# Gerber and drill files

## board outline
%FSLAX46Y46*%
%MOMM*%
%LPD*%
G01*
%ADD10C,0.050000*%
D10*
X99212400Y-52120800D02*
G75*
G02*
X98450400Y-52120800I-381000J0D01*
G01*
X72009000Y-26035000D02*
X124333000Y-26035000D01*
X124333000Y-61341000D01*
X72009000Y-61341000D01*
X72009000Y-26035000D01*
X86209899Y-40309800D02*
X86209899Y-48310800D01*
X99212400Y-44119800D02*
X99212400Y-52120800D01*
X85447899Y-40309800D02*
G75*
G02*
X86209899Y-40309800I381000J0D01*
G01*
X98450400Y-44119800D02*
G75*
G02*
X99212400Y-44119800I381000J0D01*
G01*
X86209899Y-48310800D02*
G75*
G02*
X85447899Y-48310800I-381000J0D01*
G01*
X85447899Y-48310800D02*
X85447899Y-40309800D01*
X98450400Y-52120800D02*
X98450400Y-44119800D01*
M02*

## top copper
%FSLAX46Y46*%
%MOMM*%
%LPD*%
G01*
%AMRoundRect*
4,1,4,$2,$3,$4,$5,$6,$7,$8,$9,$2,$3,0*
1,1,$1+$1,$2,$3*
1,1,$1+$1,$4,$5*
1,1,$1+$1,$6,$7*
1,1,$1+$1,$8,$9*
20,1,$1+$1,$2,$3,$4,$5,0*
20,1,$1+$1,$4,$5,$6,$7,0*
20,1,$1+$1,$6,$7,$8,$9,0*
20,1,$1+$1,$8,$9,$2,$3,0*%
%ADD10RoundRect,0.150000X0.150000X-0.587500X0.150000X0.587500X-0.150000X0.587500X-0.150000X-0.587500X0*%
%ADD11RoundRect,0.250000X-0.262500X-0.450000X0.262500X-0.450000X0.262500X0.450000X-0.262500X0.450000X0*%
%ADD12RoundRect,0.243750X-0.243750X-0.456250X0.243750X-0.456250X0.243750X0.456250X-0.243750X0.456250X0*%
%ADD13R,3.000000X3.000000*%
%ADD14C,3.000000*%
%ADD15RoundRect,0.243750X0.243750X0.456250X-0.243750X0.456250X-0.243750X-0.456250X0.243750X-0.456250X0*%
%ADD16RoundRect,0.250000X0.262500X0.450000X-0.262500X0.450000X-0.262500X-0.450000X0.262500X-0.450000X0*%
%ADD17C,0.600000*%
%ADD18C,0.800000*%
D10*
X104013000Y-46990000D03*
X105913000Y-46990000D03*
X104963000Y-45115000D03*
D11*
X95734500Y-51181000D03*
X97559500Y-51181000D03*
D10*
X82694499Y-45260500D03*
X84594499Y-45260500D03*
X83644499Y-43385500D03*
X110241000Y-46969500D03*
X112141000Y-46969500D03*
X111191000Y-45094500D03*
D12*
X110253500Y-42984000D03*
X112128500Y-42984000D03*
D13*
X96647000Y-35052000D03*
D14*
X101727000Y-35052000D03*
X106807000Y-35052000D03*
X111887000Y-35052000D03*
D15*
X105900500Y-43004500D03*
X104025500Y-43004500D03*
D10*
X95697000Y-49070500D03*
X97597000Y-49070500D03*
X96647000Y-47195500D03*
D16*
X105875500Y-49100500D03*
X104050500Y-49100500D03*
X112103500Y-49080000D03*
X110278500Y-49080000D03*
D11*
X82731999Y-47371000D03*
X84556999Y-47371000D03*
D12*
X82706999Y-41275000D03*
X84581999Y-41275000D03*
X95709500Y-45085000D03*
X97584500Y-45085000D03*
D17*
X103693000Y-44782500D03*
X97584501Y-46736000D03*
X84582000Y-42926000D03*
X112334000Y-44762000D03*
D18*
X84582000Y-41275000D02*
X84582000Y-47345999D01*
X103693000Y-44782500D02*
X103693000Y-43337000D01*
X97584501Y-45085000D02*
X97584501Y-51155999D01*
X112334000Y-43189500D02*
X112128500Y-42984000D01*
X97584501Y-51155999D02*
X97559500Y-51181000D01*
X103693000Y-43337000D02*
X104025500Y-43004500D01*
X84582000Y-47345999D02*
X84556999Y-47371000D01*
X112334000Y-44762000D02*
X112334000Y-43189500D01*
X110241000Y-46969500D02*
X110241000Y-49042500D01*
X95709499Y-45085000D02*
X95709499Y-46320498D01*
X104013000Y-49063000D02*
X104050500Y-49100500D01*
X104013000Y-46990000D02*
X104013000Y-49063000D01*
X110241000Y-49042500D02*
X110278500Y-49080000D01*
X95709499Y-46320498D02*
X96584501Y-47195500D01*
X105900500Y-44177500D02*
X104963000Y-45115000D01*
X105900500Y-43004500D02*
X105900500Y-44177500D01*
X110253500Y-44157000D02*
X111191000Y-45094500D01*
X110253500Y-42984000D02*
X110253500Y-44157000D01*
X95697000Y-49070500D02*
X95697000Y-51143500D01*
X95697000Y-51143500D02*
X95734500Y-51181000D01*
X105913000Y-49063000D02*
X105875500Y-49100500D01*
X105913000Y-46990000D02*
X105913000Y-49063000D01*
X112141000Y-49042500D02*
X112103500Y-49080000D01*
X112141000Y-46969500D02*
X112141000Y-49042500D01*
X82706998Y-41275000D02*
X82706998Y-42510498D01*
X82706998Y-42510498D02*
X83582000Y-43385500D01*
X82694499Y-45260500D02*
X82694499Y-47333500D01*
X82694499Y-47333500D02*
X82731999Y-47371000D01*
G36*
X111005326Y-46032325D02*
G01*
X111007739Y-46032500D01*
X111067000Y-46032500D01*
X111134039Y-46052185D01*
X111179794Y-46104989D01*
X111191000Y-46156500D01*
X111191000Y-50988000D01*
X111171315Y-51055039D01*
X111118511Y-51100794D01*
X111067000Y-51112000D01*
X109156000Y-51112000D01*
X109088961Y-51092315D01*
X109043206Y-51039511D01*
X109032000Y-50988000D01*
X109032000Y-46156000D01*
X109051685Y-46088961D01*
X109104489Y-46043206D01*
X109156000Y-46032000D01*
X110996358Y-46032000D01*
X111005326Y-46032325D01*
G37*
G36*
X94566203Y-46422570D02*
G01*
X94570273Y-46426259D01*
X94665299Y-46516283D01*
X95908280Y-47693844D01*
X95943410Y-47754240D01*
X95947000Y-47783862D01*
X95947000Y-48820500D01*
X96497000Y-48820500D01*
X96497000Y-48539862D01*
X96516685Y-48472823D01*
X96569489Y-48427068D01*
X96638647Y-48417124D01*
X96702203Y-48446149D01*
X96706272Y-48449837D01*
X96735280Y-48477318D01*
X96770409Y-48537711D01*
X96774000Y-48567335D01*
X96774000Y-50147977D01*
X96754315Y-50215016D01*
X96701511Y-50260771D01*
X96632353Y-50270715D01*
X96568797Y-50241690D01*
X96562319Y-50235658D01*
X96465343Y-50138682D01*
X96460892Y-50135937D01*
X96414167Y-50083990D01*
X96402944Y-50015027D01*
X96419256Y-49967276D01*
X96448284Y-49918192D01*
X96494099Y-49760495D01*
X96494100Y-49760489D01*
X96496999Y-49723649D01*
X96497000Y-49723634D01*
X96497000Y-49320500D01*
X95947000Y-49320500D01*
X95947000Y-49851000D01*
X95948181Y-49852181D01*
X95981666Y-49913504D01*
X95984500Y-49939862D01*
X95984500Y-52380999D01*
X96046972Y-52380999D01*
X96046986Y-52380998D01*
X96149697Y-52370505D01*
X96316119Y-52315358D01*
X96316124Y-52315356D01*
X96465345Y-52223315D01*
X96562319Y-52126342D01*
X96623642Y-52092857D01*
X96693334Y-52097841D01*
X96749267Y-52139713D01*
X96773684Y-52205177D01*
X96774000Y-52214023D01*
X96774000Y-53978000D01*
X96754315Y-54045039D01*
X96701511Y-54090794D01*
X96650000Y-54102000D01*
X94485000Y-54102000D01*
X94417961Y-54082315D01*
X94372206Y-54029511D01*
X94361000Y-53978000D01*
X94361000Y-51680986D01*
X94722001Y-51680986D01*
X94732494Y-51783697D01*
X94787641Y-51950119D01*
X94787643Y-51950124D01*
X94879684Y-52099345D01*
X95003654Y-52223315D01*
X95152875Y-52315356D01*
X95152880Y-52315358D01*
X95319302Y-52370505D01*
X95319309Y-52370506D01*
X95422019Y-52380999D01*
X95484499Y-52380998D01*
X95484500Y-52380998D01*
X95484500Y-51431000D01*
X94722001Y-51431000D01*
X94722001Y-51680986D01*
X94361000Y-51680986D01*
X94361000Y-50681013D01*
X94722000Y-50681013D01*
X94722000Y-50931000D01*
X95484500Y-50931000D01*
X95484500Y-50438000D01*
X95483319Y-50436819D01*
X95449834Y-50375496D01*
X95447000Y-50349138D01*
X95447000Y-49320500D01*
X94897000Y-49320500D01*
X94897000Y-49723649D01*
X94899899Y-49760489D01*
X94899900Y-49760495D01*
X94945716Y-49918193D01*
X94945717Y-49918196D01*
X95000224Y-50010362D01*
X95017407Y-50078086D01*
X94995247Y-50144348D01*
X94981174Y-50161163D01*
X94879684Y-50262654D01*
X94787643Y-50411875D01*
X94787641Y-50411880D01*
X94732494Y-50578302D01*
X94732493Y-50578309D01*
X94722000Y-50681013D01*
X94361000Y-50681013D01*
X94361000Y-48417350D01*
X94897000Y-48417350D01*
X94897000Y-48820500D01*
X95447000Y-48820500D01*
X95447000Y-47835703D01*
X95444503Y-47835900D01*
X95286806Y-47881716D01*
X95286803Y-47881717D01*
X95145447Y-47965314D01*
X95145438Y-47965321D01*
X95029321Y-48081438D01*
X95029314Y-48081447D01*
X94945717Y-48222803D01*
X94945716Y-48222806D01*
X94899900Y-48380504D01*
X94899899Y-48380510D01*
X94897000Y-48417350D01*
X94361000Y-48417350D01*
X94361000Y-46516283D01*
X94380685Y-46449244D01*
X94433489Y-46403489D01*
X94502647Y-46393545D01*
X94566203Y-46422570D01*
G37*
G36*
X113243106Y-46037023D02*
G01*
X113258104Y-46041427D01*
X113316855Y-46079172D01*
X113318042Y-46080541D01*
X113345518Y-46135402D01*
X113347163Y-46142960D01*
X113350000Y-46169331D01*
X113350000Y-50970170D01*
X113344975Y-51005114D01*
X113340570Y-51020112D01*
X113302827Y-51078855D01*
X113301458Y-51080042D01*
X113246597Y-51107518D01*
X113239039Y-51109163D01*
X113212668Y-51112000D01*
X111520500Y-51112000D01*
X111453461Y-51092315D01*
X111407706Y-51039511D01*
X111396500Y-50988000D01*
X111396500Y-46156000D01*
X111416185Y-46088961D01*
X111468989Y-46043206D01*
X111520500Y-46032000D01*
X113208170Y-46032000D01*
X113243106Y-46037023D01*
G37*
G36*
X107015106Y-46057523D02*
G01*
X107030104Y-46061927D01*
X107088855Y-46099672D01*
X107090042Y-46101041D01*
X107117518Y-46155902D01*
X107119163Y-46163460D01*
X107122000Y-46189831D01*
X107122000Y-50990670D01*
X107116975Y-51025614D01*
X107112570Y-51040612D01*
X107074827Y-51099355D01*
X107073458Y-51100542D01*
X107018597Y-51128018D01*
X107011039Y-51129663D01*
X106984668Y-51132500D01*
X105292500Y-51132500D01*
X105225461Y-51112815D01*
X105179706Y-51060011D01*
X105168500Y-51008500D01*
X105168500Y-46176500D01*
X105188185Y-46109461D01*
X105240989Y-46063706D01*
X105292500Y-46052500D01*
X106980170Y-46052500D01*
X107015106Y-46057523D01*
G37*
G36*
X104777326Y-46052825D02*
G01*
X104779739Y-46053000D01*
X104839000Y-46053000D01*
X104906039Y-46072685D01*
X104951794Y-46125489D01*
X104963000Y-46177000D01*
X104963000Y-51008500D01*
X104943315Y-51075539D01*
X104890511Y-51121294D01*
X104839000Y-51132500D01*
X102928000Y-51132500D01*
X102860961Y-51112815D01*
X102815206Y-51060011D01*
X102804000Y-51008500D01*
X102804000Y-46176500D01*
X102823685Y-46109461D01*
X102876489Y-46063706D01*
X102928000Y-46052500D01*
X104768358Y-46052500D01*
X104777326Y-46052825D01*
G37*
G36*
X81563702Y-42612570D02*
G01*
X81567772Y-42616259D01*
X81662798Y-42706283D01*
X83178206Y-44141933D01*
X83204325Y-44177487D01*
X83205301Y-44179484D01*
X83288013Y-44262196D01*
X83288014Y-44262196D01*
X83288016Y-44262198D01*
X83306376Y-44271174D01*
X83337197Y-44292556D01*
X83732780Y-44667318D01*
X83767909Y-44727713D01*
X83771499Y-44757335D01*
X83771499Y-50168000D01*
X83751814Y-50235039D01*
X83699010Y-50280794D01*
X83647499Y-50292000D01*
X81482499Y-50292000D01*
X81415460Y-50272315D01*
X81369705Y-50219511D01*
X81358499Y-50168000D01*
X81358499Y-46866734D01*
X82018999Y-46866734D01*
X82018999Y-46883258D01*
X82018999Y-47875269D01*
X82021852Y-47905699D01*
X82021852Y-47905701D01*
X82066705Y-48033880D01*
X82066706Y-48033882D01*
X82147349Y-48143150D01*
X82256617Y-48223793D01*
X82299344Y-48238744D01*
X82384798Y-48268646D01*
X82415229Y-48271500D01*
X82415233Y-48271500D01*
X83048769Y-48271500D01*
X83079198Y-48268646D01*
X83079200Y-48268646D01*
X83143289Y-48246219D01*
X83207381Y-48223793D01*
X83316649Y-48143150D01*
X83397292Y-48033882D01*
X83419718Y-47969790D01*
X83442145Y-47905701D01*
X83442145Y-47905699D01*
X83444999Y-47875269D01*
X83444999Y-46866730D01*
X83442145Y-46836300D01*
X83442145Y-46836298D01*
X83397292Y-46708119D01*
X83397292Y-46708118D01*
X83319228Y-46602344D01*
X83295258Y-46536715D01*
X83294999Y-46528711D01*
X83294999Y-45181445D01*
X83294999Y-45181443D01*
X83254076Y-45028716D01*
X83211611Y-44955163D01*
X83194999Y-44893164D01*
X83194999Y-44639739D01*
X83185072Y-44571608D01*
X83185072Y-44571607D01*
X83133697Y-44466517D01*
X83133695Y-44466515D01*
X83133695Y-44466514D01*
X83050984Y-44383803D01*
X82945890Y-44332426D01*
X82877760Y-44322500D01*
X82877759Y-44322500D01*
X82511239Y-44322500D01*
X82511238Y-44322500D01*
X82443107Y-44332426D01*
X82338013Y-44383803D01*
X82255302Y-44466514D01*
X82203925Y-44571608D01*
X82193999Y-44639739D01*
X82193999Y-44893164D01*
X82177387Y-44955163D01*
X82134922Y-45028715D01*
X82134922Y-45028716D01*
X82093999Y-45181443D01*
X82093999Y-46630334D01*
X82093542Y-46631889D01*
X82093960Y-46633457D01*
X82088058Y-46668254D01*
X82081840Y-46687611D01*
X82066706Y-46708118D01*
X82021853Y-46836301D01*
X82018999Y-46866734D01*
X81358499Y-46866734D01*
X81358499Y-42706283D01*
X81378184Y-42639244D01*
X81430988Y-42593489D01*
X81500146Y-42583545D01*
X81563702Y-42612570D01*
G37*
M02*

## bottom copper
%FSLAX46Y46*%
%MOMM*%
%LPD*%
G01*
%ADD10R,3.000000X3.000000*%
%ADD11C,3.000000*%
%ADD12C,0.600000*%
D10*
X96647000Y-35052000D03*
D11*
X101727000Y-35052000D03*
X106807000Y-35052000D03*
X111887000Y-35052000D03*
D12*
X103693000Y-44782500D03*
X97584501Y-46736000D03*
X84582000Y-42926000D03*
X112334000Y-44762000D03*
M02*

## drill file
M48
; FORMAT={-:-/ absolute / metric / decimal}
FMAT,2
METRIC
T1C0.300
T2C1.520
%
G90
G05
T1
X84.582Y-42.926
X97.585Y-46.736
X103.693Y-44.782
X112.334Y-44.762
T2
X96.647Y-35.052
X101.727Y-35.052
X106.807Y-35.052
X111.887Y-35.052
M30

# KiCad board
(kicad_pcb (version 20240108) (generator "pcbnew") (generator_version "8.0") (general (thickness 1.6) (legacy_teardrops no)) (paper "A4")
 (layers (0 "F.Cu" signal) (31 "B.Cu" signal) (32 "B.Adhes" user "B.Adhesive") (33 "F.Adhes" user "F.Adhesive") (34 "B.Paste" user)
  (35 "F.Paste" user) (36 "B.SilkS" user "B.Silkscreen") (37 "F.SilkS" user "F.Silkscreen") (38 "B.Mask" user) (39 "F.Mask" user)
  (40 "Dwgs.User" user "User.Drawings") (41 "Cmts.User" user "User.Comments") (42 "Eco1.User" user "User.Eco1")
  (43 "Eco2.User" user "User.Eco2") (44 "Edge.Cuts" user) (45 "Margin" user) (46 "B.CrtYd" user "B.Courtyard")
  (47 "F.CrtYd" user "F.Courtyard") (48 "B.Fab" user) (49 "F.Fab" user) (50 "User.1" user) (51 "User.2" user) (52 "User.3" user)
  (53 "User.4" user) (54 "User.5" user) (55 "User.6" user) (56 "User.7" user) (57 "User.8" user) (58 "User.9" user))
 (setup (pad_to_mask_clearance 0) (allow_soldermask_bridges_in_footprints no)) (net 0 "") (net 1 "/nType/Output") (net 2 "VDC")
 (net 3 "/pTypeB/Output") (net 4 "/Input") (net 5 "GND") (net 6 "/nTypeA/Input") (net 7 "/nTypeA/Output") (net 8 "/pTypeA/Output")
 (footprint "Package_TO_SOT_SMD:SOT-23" (layer "F.Cu") (at 104.963 46.0525 90)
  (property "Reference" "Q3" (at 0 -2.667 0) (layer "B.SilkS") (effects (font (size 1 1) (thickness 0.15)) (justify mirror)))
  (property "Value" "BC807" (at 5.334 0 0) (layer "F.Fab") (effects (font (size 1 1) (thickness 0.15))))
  (pad "1" smd roundrect (at -0.9375 -0.95 90) (size 1.475 0.6) (layers "F.Cu" "F.Paste" "F.Mask") (roundrect_rratio 0.25)
   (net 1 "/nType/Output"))
  (pad "2" smd roundrect (at -0.9375 0.95 90) (size 1.475 0.6) (layers "F.Cu" "F.Paste" "F.Mask") (roundrect_rratio 0.25) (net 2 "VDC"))
  (pad "3" smd roundrect (at 0.9375 0 90) (size 1.475 0.6) (layers "F.Cu" "F.Paste" "F.Mask") (roundrect_rratio 0.25)
   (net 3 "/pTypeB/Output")))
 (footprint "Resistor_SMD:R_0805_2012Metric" (layer "F.Cu") (at 96.647 51.181)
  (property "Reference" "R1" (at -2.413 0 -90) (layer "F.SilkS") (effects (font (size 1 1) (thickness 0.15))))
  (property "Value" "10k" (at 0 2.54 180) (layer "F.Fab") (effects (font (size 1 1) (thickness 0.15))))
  (pad "1" smd roundrect (at -0.9125 0) (size 1.025 1.4) (layers "F.Cu" "F.Paste" "F.Mask") (roundrect_rratio 0.243902) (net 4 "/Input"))
  (pad "2" smd roundrect (at 0.9125 0) (size 1.025 1.4) (layers "F.Cu" "F.Paste" "F.Mask") (roundrect_rratio 0.243902) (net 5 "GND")))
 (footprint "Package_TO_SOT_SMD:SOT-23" (layer "F.Cu") (at 83.644499 44.323 90)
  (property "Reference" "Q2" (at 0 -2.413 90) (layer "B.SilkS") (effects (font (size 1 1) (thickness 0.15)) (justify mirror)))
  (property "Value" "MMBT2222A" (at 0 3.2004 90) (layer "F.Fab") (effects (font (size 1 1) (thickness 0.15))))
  (pad "1" smd roundrect (at -0.9375 -0.95 90) (size 1.475 0.6) (layers "F.Cu" "F.Paste" "F.Mask") (roundrect_rratio 0.25)
   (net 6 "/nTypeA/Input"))
  (pad "2" smd roundrect (at -0.9375 0.95 90) (size 1.475 0.6) (layers "F.Cu" "F.Paste" "F.Mask") (roundrect_rratio 0.25) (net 5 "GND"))
  (pad "3" smd roundrect (at 0.9375 0 90) (size 1.475 0.6) (layers "F.Cu" "F.Paste" "F.Mask") (roundrect_rratio 0.25)
   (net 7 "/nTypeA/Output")))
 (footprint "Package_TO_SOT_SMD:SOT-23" (layer "F.Cu") (at 111.191 46.032 90)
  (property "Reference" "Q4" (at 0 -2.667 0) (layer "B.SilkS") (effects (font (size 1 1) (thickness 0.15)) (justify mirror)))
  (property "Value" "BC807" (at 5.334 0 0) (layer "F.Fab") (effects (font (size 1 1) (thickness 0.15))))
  (pad "1" smd roundrect (at -0.9375 -0.95 90) (size 1.475 0.6) (layers "F.Cu" "F.Paste" "F.Mask") (roundrect_rratio 0.25)
   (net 1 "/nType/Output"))
  (pad "2" smd roundrect (at -0.9375 0.95 90) (size 1.475 0.6) (layers "F.Cu" "F.Paste" "F.Mask") (roundrect_rratio 0.25) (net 2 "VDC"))
  (pad "3" smd roundrect (at 0.9375 0 90) (size 1.475 0.6) (layers "F.Cu" "F.Paste" "F.Mask") (roundrect_rratio 0.25)
   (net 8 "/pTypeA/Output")))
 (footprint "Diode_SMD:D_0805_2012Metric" (layer "F.Cu") (at 111.191 42.984)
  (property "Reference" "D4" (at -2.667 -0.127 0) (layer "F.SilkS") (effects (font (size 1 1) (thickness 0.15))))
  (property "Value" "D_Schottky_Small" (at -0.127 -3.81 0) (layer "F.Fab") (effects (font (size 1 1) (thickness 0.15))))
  (pad "1" smd roundrect (at -0.9375 0) (size 0.975 1.4) (layers "F.Cu" "F.Paste" "F.Mask") (roundrect_rratio 0.25) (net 8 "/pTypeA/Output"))
  (pad "2" smd roundrect (at 0.9375 0) (size 0.975 1.4) (layers "F.Cu" "F.Paste" "F.Mask") (roundrect_rratio 0.25) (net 5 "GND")))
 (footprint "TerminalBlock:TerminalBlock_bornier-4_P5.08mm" (layer "F.Cu") (at 96.647 35.052)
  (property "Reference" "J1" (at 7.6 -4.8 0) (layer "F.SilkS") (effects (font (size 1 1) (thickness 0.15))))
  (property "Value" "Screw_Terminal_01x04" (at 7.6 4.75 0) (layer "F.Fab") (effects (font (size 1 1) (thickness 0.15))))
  (pad "1" thru_hole rect (at 0 0) (size 3 3) (drill 1.52) (layers "*.Cu" "*.Mask") (remove_unused_layers no) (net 3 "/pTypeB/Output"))
  (pad "2" thru_hole circle (at 5.08 0) (size 3 3) (drill 1.52) (layers "*.Cu" "*.Mask") (remove_unused_layers no) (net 1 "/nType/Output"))
  (pad "3" thru_hole circle (at 10.16 0) (size 3 3) (drill 1.52) (layers "*.Cu" "*.Mask") (remove_unused_layers no) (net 8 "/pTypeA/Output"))
  (pad "4" thru_hole circle (at 15.24 0) (size 3 3) (drill 1.52) (layers "*.Cu" "*.Mask") (remove_unused_layers no) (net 5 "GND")))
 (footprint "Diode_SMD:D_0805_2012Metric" (layer "F.Cu") (at 104.963 43.0045 180)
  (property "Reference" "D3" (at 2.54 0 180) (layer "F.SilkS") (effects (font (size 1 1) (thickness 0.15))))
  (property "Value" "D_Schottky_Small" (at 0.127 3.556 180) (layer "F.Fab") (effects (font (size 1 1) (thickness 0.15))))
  (pad "1" smd roundrect (at -0.9375 0 180) (size 0.975 1.4) (layers "F.Cu" "F.Paste" "F.Mask") (roundrect_rratio 0.25)
   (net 3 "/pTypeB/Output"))
  (pad "2" smd roundrect (at 0.9375 0 180) (size 0.975 1.4) (layers "F.Cu" "F.Paste" "F.Mask") (roundrect_rratio 0.25) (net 5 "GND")))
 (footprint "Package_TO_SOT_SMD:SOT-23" (layer "F.Cu") (at 96.647 48.133 90)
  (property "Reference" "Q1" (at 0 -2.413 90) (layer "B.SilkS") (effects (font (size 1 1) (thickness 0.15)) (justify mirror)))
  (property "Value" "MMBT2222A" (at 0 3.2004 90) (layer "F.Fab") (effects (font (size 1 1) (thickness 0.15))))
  (pad "1" smd roundrect (at -0.9375 -0.95 90) (size 1.475 0.6) (layers "F.Cu" "F.Paste" "F.Mask") (roundrect_rratio 0.25) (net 4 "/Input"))
  (pad "2" smd roundrect (at -0.9375 0.95 90) (size 1.475 0.6) (layers "F.Cu" "F.Paste" "F.Mask") (roundrect_rratio 0.25) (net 5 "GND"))
  (pad "3" smd roundrect (at 0.9375 0 90) (size 1.475 0.6) (layers "F.Cu" "F.Paste" "F.Mask") (roundrect_rratio 0.25)
   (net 1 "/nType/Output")))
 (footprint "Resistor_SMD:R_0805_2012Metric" (layer "F.Cu") (at 104.963 49.1005 180)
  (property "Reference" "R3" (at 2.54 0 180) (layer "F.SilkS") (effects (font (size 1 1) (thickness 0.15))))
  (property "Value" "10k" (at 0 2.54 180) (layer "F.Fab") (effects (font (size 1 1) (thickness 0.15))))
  (pad "1" smd roundrect (at -0.9125 0 180) (size 1.025 1.4) (layers "F.Cu" "F.Paste" "F.Mask") (roundrect_rratio 0.243902) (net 2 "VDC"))
  (pad "2" smd roundrect (at 0.9125 0 180) (size 1.025 1.4) (layers "F.Cu" "F.Paste" "F.Mask") (roundrect_rratio 0.243902)
   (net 1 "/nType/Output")))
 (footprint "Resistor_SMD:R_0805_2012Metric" (layer "F.Cu") (at 111.191 49.08 180)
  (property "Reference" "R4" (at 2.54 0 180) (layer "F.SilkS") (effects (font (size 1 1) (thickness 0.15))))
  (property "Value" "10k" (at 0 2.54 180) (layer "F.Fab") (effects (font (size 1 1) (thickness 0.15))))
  (pad "1" smd roundrect (at -0.9125 0 180) (size 1.025 1.4) (layers "F.Cu" "F.Paste" "F.Mask") (roundrect_rratio 0.243902) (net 2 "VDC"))
  (pad "2" smd roundrect (at 0.9125 0 180) (size 1.025 1.4) (layers "F.Cu" "F.Paste" "F.Mask") (roundrect_rratio 0.243902)
   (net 1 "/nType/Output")))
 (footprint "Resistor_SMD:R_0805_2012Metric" (layer "F.Cu") (at 83.644499 47.371)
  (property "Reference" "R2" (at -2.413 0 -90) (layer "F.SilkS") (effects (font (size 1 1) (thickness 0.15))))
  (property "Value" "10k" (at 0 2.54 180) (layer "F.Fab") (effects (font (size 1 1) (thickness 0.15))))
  (pad "1" smd roundrect (at -0.9125 0) (size 1.025 1.4) (layers "F.Cu" "F.Paste" "F.Mask") (roundrect_rratio 0.243902)
   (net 6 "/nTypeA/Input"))
  (pad "2" smd roundrect (at 0.9125 0) (size 1.025 1.4) (layers "F.Cu" "F.Paste" "F.Mask") (roundrect_rratio 0.243902) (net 5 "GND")))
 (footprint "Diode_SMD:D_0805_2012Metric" (layer "F.Cu") (at 83.644499 41.275)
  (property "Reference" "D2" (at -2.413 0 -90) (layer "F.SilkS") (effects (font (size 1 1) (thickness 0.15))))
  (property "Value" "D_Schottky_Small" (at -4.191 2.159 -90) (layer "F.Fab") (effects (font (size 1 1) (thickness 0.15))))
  (pad "1" smd roundrect (at -0.9375 0) (size 0.975 1.4) (layers "F.Cu" "F.Paste" "F.Mask") (roundrect_rratio 0.25) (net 7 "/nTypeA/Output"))
  (pad "2" smd roundrect (at 0.9375 0) (size 0.975 1.4) (layers "F.Cu" "F.Paste" "F.Mask") (roundrect_rratio 0.25) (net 5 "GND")))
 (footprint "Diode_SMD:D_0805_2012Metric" (layer "F.Cu") (at 96.647 45.085)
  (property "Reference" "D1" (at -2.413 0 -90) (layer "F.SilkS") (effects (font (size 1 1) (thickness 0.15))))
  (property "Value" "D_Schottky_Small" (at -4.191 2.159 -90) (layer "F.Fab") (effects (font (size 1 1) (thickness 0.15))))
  (pad "1" smd roundrect (at -0.9375 0) (size 0.975 1.4) (layers "F.Cu" "F.Paste" "F.Mask") (roundrect_rratio 0.25) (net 1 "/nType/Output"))
  (pad "2" smd roundrect (at 0.9375 0) (size 0.975 1.4) (layers "F.Cu" "F.Paste" "F.Mask") (roundrect_rratio 0.25) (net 5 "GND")))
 (gr_arc (start 99.2124 52.1208) (mid 98.8314 52.5018) (end 98.4504 52.1208) (stroke (width 0.05) (type default)) (layer "Edge.Cuts"))
 (gr_rect (start 72.009 26.035) (end 124.333 61.341) (stroke (width 0.05) (type default)) (fill none) (layer "Edge.Cuts"))
 (gr_line (start 86.209899 40.3098) (end 86.209899 48.3108) (stroke (width 0.05) (type default)) (layer "Edge.Cuts"))
 (gr_line (start 99.2124 44.1198) (end 99.2124 52.1208) (stroke (width 0.05) (type default)) (layer "Edge.Cuts"))
 (gr_arc (start 85.447899 40.3098) (mid 85.828899 39.9288) (end 86.209899 40.3098) (stroke (width 0.05) (type default)) (layer "Edge.Cuts"))
 (gr_arc (start 98.4504 44.1198) (mid 98.8314 43.7388) (end 99.2124 44.1198) (stroke (width 0.05) (type default)) (layer "Edge.Cuts"))
 (gr_arc (start 86.209899 48.3108) (mid 85.828899 48.6918) (end 85.447899 48.3108) (stroke (width 0.05) (type default)) (layer "Edge.Cuts"))
 (gr_line (start 85.447899 48.3108) (end 85.447899 40.3098) (stroke (width 0.05) (type default)) (layer "Edge.Cuts"))
 (gr_line (start 98.4504 52.1208) (end 98.4504 44.1198) (stroke (width 0.05) (type default)) (layer "Edge.Cuts"))
 (segment (start 84.582 41.275) (end 84.582 47.345999) (width 0.8) (layer "F.Cu") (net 5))
 (segment (start 103.693 44.7825) (end 103.693 43.337) (width 0.8) (layer "F.Cu") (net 5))
 (segment (start 97.584501 45.085) (end 97.584501 51.155999) (width 0.8) (layer "F.Cu") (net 5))
 (segment (start 112.334 43.1895) (end 112.1285 42.984) (width 0.8) (layer "F.Cu") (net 5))
 (segment (start 97.584501 51.155999) (end 97.5595 51.181) (width 0.8) (layer "F.Cu") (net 5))
 (segment (start 103.693 43.337) (end 104.0255 43.0045) (width 0.8) (layer "F.Cu") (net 5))
 (segment (start 84.582 47.345999) (end 84.556999 47.371) (width 0.8) (layer "F.Cu") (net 5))
 (segment (start 112.334 44.762) (end 112.334 43.1895) (width 0.8) (layer "F.Cu") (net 5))
 (via (at 103.693 44.7825) (size 0.6) (drill 0.3) (layers "F.Cu" "B.Cu") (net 5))
 (via (at 97.584501 46.736) (size 0.6) (drill 0.3) (layers "F.Cu" "B.Cu") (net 5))
 (via (at 84.582 42.926) (size 0.6) (drill 0.3) (layers "F.Cu" "B.Cu") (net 5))
 (via (at 112.334 44.762) (size 0.6) (drill 0.3) (layers "F.Cu" "B.Cu") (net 5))
 (segment (start 110.241 46.9695) (end 110.241 49.0425) (width 0.8) (layer "F.Cu") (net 1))
 (segment (start 95.709499 45.085) (end 95.709499 46.320498) (width 0.8) (layer "F.Cu") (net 1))
 (segment (start 104.013 49.063) (end 104.0505 49.1005) (width 0.8) (layer "F.Cu") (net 1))
 (segment (start 104.013 46.99) (end 104.013 49.063) (width 0.8) (layer "F.Cu") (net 1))
 (segment (start 110.241 49.0425) (end 110.2785 49.08) (width 0.8) (layer "F.Cu") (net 1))
 (segment (start 95.709499 46.320498) (end 96.584501 47.1955) (width 0.8) (layer "F.Cu") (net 1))
 (segment (start 105.9005 44.1775) (end 104.963 45.115) (width 0.8) (layer "F.Cu") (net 3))
 (segment (start 105.9005 43.0045) (end 105.9005 44.1775) (width 0.8) (layer "F.Cu") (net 3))
 (segment (start 110.2535 44.157) (end 111.191 45.0945) (width 0.8) (layer "F.Cu") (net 8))
 (segment (start 110.2535 42.984) (end 110.2535 44.157) (width 0.8) (layer "F.Cu") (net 8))
 (segment (start 95.697 49.0705) (end 95.697 51.1435) (width 0.8) (layer "F.Cu") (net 4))
 (segment (start 95.697 51.1435) (end 95.7345 51.181) (width 0.8) (layer "F.Cu") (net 4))
 (segment (start 105.913 49.063) (end 105.8755 49.1005) (width 0.8) (layer "F.Cu") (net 2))
 (segment (start 105.913 46.99) (end 105.913 49.063) (width 0.8) (layer "F.Cu") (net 2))
 (segment (start 112.141 49.0425) (end 112.1035 49.08) (width 0.8) (layer "F.Cu") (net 2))
 (segment (start 112.141 46.9695) (end 112.141 49.0425) (width 0.8) (layer "F.Cu") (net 2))
 (segment (start 82.706998 41.275) (end 82.706998 42.510498) (width 0.8) (layer "F.Cu") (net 7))
 (segment (start 82.706998 42.510498) (end 83.582 43.3855) (width 0.8) (layer "F.Cu") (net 7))
 (segment (start 82.694499 45.2605) (end 82.694499 47.3335) (width 0.8) (layer "F.Cu") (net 6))
 (segment (start 82.694499 47.3335) (end 82.731999 47.371) (width 0.8) (layer "F.Cu") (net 6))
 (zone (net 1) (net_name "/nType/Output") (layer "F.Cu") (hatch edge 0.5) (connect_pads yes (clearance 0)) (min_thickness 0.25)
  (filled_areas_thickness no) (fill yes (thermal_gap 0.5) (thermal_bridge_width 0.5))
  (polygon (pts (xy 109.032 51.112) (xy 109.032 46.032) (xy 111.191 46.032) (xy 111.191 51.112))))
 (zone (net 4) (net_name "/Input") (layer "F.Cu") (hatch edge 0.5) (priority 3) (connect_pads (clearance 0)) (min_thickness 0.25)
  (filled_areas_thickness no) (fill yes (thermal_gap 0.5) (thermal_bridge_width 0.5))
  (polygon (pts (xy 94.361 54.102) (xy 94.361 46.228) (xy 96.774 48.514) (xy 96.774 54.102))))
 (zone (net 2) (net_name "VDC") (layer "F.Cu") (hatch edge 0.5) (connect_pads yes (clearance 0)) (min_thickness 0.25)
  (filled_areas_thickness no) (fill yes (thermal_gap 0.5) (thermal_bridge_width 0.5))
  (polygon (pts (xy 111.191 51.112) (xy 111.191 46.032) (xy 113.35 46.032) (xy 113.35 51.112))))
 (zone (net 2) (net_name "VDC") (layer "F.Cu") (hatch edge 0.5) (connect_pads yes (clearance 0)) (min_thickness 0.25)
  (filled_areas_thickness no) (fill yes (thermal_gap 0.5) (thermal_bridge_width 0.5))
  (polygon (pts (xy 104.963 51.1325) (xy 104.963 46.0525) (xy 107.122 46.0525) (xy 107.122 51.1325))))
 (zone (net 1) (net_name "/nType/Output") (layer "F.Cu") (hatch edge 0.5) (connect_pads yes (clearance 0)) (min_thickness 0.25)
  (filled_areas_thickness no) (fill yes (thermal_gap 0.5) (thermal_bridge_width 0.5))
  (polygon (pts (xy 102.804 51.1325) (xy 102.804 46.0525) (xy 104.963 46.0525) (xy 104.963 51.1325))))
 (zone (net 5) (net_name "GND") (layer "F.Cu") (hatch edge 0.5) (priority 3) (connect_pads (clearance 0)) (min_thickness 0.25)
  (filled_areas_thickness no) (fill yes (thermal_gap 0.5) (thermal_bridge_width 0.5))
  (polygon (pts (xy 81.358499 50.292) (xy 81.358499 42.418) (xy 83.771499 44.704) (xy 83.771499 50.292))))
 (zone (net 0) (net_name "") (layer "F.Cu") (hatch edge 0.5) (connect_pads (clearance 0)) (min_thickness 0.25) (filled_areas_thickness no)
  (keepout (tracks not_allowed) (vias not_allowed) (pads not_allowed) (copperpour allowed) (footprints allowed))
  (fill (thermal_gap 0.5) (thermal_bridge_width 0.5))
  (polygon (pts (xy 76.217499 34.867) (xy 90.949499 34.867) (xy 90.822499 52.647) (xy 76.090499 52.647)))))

